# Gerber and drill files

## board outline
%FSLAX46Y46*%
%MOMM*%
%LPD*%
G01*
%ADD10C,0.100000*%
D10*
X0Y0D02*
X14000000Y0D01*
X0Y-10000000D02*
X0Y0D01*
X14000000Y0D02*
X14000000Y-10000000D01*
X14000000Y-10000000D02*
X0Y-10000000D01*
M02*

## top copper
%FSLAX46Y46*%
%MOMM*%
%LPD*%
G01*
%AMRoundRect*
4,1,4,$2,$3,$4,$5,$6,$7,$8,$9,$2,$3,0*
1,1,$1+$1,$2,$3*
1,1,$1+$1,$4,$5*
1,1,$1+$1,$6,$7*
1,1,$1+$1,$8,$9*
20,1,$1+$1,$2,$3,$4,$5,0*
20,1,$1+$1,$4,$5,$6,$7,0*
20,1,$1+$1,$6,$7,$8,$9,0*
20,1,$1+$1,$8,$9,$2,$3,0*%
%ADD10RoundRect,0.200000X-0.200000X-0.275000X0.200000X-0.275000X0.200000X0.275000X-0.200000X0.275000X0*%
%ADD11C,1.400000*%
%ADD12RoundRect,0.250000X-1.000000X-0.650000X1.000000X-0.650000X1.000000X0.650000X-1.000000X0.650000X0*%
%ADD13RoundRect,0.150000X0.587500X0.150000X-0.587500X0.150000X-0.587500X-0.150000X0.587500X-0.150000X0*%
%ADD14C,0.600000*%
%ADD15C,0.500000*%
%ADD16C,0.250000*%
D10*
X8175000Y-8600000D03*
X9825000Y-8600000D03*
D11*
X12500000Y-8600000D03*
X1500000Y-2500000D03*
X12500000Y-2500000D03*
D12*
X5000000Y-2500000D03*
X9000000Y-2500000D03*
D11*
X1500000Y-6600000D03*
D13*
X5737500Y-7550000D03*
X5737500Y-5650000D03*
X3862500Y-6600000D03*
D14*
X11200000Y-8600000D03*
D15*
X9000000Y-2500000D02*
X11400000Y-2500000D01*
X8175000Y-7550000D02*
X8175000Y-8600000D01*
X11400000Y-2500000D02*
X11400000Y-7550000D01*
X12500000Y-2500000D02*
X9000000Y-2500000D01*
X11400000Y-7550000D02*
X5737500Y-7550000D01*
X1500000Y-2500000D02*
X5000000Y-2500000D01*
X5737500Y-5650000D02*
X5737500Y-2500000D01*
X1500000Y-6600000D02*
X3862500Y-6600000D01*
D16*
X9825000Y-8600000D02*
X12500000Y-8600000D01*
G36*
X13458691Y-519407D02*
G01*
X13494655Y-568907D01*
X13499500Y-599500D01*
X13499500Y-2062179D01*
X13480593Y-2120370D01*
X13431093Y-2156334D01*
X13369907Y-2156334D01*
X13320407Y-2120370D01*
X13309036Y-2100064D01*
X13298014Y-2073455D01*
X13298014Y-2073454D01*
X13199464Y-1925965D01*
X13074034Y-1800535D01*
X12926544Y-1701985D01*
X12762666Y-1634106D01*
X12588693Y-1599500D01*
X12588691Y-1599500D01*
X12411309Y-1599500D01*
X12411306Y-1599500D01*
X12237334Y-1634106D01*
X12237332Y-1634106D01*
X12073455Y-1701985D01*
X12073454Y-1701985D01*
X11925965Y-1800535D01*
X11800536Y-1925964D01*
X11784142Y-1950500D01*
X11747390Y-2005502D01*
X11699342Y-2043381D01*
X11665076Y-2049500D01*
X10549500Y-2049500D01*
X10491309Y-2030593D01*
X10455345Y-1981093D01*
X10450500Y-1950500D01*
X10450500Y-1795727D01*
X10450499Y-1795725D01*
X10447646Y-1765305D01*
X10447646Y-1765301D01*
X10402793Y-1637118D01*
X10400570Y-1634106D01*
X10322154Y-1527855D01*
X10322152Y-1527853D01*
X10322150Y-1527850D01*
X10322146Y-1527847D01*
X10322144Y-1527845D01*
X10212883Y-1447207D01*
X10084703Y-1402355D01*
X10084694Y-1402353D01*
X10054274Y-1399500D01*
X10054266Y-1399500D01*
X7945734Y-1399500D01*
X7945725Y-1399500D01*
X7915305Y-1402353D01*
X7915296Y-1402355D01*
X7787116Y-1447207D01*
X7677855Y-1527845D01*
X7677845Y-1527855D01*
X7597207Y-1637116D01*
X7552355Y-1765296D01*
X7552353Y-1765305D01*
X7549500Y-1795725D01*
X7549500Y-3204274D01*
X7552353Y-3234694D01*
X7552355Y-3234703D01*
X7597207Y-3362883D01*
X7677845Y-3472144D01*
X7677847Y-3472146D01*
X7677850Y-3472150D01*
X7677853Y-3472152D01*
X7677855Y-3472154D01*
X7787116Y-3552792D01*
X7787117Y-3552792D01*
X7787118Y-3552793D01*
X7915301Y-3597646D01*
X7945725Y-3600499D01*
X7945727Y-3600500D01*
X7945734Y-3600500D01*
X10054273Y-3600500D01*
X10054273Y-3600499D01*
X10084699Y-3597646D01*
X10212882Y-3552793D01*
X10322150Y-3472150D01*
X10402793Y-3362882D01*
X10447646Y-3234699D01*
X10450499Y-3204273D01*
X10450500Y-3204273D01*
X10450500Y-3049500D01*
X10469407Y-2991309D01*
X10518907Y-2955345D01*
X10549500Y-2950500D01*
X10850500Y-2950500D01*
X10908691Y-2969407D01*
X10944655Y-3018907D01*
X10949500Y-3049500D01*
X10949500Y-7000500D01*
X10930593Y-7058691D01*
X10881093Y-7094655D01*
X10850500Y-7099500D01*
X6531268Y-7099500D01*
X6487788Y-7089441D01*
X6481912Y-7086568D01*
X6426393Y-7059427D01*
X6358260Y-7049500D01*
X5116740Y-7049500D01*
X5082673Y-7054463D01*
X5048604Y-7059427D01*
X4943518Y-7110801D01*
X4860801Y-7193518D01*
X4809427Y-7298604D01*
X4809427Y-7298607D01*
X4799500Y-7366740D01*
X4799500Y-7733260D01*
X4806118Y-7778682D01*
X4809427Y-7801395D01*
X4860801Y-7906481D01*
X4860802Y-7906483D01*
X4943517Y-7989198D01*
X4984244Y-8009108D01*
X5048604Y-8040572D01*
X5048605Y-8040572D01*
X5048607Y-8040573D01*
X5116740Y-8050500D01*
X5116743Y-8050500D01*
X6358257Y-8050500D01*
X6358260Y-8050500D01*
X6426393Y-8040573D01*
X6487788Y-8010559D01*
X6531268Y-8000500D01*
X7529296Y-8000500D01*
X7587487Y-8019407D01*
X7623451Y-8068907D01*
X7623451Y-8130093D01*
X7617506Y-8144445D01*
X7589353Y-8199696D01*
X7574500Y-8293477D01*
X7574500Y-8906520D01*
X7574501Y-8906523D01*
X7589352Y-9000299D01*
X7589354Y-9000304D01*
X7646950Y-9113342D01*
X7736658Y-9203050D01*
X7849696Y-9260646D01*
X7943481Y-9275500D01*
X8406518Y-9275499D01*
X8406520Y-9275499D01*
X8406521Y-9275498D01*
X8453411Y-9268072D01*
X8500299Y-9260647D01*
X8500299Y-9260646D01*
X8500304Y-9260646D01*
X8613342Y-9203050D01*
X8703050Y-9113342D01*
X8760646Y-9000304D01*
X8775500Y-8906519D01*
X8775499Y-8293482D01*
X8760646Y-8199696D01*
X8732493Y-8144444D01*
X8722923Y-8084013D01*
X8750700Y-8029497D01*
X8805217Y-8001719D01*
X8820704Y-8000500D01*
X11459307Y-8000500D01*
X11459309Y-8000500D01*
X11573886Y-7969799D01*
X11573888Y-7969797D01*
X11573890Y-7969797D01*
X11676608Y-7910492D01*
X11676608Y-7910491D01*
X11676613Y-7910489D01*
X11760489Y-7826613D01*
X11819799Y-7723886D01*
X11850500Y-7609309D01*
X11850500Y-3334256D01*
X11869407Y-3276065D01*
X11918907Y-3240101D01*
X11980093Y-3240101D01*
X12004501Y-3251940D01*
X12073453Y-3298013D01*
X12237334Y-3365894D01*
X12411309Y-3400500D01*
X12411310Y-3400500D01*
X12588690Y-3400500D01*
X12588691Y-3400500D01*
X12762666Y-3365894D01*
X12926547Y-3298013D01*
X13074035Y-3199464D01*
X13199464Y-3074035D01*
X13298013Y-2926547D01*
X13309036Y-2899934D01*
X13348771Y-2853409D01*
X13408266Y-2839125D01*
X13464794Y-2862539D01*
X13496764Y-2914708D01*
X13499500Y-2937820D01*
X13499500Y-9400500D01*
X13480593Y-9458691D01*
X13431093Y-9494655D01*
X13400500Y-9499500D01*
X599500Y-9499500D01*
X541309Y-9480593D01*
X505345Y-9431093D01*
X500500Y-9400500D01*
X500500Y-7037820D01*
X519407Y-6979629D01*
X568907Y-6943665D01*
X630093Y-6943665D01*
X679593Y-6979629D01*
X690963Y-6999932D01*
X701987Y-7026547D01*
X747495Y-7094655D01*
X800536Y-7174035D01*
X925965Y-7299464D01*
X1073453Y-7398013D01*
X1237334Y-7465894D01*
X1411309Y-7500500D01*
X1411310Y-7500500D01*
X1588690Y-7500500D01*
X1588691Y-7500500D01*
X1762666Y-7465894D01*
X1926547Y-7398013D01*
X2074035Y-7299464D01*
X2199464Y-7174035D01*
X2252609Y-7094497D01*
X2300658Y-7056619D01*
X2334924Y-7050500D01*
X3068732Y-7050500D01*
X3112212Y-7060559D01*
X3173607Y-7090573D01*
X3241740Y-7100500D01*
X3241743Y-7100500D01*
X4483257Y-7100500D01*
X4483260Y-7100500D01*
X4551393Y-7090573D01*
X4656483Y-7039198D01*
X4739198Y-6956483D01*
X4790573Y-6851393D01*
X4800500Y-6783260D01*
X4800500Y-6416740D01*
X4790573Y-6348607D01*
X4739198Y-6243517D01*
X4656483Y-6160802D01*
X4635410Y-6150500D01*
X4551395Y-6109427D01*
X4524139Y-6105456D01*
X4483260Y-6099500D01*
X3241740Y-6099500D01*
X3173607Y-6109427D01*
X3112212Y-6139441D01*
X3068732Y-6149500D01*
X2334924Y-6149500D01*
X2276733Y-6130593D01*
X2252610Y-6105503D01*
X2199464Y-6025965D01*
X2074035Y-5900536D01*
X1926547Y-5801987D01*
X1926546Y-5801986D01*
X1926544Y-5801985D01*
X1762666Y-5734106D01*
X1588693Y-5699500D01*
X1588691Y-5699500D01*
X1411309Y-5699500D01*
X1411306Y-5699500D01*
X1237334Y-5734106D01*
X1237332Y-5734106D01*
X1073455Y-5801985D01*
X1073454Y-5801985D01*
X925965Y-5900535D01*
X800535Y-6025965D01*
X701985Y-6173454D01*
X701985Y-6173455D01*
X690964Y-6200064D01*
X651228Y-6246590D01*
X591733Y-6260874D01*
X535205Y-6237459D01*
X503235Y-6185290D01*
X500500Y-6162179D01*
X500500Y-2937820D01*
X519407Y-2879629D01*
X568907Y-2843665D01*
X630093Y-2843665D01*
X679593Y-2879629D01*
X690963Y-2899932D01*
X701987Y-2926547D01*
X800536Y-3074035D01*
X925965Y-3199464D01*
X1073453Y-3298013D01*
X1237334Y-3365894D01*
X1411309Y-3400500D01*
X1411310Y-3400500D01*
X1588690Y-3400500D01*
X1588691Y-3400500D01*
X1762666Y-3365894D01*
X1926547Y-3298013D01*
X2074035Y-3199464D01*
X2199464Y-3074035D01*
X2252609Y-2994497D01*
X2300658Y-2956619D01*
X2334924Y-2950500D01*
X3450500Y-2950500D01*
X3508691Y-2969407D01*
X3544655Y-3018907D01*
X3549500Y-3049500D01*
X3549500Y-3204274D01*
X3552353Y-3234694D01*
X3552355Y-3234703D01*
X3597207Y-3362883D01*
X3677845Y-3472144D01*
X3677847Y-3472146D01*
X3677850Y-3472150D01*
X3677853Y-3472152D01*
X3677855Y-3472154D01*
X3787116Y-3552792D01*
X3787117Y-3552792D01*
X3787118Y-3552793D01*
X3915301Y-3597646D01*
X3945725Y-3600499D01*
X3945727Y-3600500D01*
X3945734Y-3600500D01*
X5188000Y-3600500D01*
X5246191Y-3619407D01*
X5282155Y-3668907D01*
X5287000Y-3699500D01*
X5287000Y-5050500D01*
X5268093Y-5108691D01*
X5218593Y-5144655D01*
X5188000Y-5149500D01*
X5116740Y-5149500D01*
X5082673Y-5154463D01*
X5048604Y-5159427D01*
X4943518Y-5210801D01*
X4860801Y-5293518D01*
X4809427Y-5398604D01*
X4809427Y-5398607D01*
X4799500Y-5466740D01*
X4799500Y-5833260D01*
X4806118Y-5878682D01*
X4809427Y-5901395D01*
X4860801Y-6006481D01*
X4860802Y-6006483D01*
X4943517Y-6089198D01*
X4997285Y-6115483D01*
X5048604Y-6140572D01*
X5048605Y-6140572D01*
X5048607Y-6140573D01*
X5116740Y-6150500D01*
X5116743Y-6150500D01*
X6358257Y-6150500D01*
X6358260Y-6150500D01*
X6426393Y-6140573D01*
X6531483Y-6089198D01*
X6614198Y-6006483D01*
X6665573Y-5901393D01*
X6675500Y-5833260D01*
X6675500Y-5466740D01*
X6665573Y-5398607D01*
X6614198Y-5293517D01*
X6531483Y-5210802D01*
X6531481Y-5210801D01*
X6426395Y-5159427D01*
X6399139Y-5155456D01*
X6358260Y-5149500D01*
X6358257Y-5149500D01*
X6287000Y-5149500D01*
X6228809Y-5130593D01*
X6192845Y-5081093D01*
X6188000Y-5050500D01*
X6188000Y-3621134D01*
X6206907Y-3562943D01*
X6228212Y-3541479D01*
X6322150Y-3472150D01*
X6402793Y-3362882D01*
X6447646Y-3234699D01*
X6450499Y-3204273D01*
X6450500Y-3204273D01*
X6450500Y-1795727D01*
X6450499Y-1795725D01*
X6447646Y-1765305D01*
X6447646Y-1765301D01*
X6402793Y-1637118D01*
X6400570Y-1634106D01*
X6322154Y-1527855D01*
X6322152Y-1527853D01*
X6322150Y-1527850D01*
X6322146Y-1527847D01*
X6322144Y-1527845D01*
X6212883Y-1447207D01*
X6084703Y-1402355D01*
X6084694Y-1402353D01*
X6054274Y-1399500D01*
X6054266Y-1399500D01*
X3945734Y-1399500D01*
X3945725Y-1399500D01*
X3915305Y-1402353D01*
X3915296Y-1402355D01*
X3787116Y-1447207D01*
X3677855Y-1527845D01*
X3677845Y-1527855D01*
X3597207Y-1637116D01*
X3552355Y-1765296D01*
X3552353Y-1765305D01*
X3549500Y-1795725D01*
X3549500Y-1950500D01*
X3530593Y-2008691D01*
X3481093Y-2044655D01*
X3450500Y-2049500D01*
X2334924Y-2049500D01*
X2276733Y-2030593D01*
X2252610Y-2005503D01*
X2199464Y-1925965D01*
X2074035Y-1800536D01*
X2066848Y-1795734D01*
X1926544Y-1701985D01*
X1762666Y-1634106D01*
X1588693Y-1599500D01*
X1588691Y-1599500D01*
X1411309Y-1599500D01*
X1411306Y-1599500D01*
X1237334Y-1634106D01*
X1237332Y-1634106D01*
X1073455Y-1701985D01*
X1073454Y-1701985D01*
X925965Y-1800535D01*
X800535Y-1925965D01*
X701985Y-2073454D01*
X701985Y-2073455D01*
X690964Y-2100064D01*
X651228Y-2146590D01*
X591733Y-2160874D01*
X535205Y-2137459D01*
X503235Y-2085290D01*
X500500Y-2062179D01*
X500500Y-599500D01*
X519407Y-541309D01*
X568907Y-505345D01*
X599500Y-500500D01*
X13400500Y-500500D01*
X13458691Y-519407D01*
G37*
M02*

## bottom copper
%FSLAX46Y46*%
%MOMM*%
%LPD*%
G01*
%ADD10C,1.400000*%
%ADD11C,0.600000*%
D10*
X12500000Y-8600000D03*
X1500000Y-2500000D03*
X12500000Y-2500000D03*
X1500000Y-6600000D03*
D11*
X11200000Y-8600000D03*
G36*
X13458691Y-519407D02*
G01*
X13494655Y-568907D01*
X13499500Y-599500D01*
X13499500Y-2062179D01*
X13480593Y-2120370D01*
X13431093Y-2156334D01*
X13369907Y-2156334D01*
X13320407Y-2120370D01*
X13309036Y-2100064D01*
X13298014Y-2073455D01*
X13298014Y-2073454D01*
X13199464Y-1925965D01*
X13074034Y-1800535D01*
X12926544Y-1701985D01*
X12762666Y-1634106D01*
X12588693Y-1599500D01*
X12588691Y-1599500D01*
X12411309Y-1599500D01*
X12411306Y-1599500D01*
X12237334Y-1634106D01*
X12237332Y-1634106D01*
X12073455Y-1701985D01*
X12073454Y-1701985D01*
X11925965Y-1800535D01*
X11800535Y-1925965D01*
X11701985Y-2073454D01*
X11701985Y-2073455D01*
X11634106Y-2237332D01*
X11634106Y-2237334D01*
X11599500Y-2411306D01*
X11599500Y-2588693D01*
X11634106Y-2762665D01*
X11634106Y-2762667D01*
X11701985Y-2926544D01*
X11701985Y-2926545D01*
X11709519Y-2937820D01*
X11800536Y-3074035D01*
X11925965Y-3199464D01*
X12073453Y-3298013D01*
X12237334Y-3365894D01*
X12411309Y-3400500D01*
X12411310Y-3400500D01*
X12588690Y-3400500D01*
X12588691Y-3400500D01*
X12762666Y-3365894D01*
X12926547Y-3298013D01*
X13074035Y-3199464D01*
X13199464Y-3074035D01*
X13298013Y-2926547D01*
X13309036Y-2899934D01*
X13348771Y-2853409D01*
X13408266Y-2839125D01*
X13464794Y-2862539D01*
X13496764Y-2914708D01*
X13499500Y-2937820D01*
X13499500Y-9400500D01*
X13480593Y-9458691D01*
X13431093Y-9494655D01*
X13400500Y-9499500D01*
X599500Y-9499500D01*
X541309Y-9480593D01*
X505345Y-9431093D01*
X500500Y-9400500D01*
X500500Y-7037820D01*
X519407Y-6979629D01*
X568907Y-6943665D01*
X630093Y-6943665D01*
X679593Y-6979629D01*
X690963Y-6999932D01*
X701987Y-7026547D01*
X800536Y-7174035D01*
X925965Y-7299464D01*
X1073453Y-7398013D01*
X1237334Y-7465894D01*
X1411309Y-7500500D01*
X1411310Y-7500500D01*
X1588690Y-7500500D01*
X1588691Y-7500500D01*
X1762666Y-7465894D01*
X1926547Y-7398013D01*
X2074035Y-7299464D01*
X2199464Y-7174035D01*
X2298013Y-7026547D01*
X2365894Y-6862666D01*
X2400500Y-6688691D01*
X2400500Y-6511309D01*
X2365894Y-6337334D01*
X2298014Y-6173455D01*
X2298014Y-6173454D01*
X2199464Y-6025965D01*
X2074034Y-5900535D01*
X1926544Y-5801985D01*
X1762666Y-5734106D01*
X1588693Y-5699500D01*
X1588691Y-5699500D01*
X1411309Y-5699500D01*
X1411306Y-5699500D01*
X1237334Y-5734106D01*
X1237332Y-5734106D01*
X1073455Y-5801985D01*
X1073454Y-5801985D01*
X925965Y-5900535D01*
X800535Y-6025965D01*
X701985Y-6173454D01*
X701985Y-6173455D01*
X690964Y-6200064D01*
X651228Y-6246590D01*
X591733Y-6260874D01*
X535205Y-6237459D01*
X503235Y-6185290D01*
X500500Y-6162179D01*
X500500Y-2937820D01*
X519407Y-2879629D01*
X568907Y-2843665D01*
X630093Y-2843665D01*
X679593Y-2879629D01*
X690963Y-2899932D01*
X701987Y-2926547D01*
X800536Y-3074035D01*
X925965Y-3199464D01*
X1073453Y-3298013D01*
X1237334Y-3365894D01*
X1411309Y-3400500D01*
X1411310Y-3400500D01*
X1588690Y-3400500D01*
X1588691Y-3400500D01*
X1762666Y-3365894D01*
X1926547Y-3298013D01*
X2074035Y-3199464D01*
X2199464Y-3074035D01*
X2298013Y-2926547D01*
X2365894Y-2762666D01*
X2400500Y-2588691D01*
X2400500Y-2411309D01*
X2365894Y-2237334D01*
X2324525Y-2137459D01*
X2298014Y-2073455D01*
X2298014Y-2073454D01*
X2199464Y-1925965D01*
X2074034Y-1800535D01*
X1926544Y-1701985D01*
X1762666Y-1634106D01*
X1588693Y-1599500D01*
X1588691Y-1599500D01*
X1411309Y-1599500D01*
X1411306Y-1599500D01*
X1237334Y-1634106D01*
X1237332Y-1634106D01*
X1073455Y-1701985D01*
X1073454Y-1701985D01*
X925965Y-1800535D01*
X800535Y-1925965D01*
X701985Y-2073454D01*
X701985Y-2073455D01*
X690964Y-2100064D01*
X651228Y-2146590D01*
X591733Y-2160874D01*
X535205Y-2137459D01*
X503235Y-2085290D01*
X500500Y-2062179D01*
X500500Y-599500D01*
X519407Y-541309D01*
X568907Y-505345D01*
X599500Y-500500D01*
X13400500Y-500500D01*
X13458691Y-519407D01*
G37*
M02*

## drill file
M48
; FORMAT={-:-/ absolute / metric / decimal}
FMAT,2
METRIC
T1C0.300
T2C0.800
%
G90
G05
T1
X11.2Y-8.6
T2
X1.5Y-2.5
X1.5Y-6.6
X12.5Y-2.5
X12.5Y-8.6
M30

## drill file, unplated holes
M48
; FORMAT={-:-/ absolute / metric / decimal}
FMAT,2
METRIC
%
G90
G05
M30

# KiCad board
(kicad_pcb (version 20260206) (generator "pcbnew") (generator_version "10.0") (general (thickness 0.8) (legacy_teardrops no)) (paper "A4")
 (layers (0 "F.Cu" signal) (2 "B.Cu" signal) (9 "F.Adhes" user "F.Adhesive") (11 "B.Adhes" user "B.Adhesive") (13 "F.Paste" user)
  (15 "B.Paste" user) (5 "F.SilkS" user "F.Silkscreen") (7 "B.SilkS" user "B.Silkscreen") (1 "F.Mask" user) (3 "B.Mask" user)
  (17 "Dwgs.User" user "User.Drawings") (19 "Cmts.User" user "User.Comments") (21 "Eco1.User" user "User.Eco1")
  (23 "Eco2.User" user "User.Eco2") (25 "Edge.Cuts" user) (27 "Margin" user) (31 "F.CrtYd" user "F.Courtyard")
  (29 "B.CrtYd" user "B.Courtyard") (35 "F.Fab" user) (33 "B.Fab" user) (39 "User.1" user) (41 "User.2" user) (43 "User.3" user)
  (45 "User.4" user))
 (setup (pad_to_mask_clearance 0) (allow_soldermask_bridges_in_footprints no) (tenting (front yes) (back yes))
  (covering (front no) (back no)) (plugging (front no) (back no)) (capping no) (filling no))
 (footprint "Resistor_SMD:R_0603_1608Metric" (layer "F.Cu") (at 9 8.6)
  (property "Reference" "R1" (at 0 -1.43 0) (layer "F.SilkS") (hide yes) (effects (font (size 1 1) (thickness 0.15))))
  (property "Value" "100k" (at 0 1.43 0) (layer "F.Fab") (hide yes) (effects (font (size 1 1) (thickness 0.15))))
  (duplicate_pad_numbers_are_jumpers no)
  (pad "1" smd roundrect (at -0.825 0) (size 0.8 0.95) (layers "F.Cu" "F.Mask" "F.Paste") (roundrect_rratio 0.25) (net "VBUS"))
  (pad "2" smd roundrect (at 0.825 0) (size 0.8 0.95) (layers "F.Cu" "F.Mask" "F.Paste") (roundrect_rratio 0.25) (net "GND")
   (zone_connect 2)))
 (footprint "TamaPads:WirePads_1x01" (layer "F.Cu") (at 12.5 8.6)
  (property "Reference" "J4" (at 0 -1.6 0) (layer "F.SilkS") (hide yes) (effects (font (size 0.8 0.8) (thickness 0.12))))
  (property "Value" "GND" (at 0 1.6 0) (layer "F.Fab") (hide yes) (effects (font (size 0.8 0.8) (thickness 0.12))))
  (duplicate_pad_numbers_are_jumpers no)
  (pad "1" thru_hole circle (at 0 0) (size 1.4 1.4) (drill 0.8) (layers "*.Cu" "*.Mask") (remove_unused_layers no) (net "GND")
   (zone_connect 2)))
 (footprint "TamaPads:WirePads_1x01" (layer "F.Cu") (at 1.5 2.5)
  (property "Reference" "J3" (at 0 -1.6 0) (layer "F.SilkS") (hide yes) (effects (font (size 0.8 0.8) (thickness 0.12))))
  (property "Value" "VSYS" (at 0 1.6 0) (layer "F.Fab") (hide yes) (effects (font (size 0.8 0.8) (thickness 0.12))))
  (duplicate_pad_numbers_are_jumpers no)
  (pad "1" thru_hole circle (at 0 0) (size 1.4 1.4) (drill 0.8) (layers "*.Cu" "*.Mask") (remove_unused_layers no) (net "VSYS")))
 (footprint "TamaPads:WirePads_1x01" (layer "F.Cu") (at 12.5 2.5)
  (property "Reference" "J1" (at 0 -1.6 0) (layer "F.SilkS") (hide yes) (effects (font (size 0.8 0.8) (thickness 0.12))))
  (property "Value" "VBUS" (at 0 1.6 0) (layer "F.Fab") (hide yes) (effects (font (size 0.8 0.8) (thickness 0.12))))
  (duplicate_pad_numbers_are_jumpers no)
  (pad "1" thru_hole circle (at 0 0) (size 1.4 1.4) (drill 0.8) (layers "*.Cu" "*.Mask") (remove_unused_layers no) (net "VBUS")))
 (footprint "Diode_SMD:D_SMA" (layer "F.Cu") (at 7 2.5)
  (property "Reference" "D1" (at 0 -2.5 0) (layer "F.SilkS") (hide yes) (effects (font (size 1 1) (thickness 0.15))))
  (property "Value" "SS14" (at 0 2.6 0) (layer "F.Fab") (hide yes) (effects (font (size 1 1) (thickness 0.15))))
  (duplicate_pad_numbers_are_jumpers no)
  (pad "1" smd roundrect (at -2 0) (size 2.5 1.8) (layers "F.Cu" "F.Mask" "F.Paste") (roundrect_rratio 0.1388888889) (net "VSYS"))
  (pad "2" smd roundrect (at 2 0) (size 2.5 1.8) (layers "F.Cu" "F.Mask" "F.Paste") (roundrect_rratio 0.1388888889) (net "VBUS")))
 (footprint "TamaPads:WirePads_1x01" (layer "F.Cu") (at 1.5 6.6)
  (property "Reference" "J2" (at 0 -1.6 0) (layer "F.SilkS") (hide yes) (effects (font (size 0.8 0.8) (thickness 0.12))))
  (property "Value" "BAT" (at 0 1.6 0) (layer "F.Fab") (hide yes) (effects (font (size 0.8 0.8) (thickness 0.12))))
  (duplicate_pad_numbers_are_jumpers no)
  (pad "1" thru_hole circle (at 0 0) (size 1.4 1.4) (drill 0.8) (layers "*.Cu" "*.Mask") (remove_unused_layers no) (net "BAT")))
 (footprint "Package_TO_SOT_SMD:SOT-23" (layer "F.Cu") (at 4.8 6.6 180)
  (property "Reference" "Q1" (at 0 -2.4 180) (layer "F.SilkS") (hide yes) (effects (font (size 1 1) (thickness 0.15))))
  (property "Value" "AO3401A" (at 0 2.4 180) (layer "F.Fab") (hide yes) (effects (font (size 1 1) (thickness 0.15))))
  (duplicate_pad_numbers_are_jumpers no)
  (pad "1" smd roundrect (at -0.9375 -0.95 180) (size 1.475 0.6) (layers "F.Cu" "F.Mask" "F.Paste") (roundrect_rratio 0.25) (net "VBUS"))
  (pad "2" smd roundrect (at -0.9375 0.95 180) (size 1.475 0.6) (layers "F.Cu" "F.Mask" "F.Paste") (roundrect_rratio 0.25) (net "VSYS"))
  (pad "3" smd roundrect (at 0.9375 0 180) (size 1.475 0.6) (layers "F.Cu" "F.Mask" "F.Paste") (roundrect_rratio 0.25) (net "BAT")))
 (gr_line (start 0 0) (end 14 0) (stroke (width 0.1) (type default)) (layer "Edge.Cuts"))
 (gr_line (start 0 10) (end 0 0) (stroke (width 0.1) (type default)) (layer "Edge.Cuts"))
 (gr_line (start 14 0) (end 14 10) (stroke (width 0.1) (type default)) (layer "Edge.Cuts"))
 (gr_line (start 14 10) (end 0 10) (stroke (width 0.1) (type default)) (layer "Edge.Cuts"))
 (segment (start 9 2.5) (end 11.4 2.5) (width 0.5) (layer "F.Cu") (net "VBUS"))
 (segment (start 8.175 7.55) (end 8.175 8.6) (width 0.5) (layer "F.Cu") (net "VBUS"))
 (segment (start 11.4 2.5) (end 11.4 7.55) (width 0.5) (layer "F.Cu") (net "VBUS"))
 (segment (start 12.5 2.5) (end 9 2.5) (width 0.5) (layer "F.Cu") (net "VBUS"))
 (segment (start 11.4 7.55) (end 5.7375 7.55) (width 0.5) (layer "F.Cu") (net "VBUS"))
 (segment (start 1.5 2.5) (end 5 2.5) (width 0.5) (layer "F.Cu") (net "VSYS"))
 (segment (start 5.7375 5.65) (end 5.7375 2.5) (width 0.5) (layer "F.Cu") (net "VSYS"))
 (segment (start 1.5 6.6) (end 3.8625 6.6) (width 0.5) (layer "F.Cu") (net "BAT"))
 (segment (start 9.825 8.6) (end 12.5 8.6) (width 0.25) (layer "F.Cu") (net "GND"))
 (via (at 11.2 8.6) (size 0.6) (drill 0.3) (layers "F.Cu" "B.Cu") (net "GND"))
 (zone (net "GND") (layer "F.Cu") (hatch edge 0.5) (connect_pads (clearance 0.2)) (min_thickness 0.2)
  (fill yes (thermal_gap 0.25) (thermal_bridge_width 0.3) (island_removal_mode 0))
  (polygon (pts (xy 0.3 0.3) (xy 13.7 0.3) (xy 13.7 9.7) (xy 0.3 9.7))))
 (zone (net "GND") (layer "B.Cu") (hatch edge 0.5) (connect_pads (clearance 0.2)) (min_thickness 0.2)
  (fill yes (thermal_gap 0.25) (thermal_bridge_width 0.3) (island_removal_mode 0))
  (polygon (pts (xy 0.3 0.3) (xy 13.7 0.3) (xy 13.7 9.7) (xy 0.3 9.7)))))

